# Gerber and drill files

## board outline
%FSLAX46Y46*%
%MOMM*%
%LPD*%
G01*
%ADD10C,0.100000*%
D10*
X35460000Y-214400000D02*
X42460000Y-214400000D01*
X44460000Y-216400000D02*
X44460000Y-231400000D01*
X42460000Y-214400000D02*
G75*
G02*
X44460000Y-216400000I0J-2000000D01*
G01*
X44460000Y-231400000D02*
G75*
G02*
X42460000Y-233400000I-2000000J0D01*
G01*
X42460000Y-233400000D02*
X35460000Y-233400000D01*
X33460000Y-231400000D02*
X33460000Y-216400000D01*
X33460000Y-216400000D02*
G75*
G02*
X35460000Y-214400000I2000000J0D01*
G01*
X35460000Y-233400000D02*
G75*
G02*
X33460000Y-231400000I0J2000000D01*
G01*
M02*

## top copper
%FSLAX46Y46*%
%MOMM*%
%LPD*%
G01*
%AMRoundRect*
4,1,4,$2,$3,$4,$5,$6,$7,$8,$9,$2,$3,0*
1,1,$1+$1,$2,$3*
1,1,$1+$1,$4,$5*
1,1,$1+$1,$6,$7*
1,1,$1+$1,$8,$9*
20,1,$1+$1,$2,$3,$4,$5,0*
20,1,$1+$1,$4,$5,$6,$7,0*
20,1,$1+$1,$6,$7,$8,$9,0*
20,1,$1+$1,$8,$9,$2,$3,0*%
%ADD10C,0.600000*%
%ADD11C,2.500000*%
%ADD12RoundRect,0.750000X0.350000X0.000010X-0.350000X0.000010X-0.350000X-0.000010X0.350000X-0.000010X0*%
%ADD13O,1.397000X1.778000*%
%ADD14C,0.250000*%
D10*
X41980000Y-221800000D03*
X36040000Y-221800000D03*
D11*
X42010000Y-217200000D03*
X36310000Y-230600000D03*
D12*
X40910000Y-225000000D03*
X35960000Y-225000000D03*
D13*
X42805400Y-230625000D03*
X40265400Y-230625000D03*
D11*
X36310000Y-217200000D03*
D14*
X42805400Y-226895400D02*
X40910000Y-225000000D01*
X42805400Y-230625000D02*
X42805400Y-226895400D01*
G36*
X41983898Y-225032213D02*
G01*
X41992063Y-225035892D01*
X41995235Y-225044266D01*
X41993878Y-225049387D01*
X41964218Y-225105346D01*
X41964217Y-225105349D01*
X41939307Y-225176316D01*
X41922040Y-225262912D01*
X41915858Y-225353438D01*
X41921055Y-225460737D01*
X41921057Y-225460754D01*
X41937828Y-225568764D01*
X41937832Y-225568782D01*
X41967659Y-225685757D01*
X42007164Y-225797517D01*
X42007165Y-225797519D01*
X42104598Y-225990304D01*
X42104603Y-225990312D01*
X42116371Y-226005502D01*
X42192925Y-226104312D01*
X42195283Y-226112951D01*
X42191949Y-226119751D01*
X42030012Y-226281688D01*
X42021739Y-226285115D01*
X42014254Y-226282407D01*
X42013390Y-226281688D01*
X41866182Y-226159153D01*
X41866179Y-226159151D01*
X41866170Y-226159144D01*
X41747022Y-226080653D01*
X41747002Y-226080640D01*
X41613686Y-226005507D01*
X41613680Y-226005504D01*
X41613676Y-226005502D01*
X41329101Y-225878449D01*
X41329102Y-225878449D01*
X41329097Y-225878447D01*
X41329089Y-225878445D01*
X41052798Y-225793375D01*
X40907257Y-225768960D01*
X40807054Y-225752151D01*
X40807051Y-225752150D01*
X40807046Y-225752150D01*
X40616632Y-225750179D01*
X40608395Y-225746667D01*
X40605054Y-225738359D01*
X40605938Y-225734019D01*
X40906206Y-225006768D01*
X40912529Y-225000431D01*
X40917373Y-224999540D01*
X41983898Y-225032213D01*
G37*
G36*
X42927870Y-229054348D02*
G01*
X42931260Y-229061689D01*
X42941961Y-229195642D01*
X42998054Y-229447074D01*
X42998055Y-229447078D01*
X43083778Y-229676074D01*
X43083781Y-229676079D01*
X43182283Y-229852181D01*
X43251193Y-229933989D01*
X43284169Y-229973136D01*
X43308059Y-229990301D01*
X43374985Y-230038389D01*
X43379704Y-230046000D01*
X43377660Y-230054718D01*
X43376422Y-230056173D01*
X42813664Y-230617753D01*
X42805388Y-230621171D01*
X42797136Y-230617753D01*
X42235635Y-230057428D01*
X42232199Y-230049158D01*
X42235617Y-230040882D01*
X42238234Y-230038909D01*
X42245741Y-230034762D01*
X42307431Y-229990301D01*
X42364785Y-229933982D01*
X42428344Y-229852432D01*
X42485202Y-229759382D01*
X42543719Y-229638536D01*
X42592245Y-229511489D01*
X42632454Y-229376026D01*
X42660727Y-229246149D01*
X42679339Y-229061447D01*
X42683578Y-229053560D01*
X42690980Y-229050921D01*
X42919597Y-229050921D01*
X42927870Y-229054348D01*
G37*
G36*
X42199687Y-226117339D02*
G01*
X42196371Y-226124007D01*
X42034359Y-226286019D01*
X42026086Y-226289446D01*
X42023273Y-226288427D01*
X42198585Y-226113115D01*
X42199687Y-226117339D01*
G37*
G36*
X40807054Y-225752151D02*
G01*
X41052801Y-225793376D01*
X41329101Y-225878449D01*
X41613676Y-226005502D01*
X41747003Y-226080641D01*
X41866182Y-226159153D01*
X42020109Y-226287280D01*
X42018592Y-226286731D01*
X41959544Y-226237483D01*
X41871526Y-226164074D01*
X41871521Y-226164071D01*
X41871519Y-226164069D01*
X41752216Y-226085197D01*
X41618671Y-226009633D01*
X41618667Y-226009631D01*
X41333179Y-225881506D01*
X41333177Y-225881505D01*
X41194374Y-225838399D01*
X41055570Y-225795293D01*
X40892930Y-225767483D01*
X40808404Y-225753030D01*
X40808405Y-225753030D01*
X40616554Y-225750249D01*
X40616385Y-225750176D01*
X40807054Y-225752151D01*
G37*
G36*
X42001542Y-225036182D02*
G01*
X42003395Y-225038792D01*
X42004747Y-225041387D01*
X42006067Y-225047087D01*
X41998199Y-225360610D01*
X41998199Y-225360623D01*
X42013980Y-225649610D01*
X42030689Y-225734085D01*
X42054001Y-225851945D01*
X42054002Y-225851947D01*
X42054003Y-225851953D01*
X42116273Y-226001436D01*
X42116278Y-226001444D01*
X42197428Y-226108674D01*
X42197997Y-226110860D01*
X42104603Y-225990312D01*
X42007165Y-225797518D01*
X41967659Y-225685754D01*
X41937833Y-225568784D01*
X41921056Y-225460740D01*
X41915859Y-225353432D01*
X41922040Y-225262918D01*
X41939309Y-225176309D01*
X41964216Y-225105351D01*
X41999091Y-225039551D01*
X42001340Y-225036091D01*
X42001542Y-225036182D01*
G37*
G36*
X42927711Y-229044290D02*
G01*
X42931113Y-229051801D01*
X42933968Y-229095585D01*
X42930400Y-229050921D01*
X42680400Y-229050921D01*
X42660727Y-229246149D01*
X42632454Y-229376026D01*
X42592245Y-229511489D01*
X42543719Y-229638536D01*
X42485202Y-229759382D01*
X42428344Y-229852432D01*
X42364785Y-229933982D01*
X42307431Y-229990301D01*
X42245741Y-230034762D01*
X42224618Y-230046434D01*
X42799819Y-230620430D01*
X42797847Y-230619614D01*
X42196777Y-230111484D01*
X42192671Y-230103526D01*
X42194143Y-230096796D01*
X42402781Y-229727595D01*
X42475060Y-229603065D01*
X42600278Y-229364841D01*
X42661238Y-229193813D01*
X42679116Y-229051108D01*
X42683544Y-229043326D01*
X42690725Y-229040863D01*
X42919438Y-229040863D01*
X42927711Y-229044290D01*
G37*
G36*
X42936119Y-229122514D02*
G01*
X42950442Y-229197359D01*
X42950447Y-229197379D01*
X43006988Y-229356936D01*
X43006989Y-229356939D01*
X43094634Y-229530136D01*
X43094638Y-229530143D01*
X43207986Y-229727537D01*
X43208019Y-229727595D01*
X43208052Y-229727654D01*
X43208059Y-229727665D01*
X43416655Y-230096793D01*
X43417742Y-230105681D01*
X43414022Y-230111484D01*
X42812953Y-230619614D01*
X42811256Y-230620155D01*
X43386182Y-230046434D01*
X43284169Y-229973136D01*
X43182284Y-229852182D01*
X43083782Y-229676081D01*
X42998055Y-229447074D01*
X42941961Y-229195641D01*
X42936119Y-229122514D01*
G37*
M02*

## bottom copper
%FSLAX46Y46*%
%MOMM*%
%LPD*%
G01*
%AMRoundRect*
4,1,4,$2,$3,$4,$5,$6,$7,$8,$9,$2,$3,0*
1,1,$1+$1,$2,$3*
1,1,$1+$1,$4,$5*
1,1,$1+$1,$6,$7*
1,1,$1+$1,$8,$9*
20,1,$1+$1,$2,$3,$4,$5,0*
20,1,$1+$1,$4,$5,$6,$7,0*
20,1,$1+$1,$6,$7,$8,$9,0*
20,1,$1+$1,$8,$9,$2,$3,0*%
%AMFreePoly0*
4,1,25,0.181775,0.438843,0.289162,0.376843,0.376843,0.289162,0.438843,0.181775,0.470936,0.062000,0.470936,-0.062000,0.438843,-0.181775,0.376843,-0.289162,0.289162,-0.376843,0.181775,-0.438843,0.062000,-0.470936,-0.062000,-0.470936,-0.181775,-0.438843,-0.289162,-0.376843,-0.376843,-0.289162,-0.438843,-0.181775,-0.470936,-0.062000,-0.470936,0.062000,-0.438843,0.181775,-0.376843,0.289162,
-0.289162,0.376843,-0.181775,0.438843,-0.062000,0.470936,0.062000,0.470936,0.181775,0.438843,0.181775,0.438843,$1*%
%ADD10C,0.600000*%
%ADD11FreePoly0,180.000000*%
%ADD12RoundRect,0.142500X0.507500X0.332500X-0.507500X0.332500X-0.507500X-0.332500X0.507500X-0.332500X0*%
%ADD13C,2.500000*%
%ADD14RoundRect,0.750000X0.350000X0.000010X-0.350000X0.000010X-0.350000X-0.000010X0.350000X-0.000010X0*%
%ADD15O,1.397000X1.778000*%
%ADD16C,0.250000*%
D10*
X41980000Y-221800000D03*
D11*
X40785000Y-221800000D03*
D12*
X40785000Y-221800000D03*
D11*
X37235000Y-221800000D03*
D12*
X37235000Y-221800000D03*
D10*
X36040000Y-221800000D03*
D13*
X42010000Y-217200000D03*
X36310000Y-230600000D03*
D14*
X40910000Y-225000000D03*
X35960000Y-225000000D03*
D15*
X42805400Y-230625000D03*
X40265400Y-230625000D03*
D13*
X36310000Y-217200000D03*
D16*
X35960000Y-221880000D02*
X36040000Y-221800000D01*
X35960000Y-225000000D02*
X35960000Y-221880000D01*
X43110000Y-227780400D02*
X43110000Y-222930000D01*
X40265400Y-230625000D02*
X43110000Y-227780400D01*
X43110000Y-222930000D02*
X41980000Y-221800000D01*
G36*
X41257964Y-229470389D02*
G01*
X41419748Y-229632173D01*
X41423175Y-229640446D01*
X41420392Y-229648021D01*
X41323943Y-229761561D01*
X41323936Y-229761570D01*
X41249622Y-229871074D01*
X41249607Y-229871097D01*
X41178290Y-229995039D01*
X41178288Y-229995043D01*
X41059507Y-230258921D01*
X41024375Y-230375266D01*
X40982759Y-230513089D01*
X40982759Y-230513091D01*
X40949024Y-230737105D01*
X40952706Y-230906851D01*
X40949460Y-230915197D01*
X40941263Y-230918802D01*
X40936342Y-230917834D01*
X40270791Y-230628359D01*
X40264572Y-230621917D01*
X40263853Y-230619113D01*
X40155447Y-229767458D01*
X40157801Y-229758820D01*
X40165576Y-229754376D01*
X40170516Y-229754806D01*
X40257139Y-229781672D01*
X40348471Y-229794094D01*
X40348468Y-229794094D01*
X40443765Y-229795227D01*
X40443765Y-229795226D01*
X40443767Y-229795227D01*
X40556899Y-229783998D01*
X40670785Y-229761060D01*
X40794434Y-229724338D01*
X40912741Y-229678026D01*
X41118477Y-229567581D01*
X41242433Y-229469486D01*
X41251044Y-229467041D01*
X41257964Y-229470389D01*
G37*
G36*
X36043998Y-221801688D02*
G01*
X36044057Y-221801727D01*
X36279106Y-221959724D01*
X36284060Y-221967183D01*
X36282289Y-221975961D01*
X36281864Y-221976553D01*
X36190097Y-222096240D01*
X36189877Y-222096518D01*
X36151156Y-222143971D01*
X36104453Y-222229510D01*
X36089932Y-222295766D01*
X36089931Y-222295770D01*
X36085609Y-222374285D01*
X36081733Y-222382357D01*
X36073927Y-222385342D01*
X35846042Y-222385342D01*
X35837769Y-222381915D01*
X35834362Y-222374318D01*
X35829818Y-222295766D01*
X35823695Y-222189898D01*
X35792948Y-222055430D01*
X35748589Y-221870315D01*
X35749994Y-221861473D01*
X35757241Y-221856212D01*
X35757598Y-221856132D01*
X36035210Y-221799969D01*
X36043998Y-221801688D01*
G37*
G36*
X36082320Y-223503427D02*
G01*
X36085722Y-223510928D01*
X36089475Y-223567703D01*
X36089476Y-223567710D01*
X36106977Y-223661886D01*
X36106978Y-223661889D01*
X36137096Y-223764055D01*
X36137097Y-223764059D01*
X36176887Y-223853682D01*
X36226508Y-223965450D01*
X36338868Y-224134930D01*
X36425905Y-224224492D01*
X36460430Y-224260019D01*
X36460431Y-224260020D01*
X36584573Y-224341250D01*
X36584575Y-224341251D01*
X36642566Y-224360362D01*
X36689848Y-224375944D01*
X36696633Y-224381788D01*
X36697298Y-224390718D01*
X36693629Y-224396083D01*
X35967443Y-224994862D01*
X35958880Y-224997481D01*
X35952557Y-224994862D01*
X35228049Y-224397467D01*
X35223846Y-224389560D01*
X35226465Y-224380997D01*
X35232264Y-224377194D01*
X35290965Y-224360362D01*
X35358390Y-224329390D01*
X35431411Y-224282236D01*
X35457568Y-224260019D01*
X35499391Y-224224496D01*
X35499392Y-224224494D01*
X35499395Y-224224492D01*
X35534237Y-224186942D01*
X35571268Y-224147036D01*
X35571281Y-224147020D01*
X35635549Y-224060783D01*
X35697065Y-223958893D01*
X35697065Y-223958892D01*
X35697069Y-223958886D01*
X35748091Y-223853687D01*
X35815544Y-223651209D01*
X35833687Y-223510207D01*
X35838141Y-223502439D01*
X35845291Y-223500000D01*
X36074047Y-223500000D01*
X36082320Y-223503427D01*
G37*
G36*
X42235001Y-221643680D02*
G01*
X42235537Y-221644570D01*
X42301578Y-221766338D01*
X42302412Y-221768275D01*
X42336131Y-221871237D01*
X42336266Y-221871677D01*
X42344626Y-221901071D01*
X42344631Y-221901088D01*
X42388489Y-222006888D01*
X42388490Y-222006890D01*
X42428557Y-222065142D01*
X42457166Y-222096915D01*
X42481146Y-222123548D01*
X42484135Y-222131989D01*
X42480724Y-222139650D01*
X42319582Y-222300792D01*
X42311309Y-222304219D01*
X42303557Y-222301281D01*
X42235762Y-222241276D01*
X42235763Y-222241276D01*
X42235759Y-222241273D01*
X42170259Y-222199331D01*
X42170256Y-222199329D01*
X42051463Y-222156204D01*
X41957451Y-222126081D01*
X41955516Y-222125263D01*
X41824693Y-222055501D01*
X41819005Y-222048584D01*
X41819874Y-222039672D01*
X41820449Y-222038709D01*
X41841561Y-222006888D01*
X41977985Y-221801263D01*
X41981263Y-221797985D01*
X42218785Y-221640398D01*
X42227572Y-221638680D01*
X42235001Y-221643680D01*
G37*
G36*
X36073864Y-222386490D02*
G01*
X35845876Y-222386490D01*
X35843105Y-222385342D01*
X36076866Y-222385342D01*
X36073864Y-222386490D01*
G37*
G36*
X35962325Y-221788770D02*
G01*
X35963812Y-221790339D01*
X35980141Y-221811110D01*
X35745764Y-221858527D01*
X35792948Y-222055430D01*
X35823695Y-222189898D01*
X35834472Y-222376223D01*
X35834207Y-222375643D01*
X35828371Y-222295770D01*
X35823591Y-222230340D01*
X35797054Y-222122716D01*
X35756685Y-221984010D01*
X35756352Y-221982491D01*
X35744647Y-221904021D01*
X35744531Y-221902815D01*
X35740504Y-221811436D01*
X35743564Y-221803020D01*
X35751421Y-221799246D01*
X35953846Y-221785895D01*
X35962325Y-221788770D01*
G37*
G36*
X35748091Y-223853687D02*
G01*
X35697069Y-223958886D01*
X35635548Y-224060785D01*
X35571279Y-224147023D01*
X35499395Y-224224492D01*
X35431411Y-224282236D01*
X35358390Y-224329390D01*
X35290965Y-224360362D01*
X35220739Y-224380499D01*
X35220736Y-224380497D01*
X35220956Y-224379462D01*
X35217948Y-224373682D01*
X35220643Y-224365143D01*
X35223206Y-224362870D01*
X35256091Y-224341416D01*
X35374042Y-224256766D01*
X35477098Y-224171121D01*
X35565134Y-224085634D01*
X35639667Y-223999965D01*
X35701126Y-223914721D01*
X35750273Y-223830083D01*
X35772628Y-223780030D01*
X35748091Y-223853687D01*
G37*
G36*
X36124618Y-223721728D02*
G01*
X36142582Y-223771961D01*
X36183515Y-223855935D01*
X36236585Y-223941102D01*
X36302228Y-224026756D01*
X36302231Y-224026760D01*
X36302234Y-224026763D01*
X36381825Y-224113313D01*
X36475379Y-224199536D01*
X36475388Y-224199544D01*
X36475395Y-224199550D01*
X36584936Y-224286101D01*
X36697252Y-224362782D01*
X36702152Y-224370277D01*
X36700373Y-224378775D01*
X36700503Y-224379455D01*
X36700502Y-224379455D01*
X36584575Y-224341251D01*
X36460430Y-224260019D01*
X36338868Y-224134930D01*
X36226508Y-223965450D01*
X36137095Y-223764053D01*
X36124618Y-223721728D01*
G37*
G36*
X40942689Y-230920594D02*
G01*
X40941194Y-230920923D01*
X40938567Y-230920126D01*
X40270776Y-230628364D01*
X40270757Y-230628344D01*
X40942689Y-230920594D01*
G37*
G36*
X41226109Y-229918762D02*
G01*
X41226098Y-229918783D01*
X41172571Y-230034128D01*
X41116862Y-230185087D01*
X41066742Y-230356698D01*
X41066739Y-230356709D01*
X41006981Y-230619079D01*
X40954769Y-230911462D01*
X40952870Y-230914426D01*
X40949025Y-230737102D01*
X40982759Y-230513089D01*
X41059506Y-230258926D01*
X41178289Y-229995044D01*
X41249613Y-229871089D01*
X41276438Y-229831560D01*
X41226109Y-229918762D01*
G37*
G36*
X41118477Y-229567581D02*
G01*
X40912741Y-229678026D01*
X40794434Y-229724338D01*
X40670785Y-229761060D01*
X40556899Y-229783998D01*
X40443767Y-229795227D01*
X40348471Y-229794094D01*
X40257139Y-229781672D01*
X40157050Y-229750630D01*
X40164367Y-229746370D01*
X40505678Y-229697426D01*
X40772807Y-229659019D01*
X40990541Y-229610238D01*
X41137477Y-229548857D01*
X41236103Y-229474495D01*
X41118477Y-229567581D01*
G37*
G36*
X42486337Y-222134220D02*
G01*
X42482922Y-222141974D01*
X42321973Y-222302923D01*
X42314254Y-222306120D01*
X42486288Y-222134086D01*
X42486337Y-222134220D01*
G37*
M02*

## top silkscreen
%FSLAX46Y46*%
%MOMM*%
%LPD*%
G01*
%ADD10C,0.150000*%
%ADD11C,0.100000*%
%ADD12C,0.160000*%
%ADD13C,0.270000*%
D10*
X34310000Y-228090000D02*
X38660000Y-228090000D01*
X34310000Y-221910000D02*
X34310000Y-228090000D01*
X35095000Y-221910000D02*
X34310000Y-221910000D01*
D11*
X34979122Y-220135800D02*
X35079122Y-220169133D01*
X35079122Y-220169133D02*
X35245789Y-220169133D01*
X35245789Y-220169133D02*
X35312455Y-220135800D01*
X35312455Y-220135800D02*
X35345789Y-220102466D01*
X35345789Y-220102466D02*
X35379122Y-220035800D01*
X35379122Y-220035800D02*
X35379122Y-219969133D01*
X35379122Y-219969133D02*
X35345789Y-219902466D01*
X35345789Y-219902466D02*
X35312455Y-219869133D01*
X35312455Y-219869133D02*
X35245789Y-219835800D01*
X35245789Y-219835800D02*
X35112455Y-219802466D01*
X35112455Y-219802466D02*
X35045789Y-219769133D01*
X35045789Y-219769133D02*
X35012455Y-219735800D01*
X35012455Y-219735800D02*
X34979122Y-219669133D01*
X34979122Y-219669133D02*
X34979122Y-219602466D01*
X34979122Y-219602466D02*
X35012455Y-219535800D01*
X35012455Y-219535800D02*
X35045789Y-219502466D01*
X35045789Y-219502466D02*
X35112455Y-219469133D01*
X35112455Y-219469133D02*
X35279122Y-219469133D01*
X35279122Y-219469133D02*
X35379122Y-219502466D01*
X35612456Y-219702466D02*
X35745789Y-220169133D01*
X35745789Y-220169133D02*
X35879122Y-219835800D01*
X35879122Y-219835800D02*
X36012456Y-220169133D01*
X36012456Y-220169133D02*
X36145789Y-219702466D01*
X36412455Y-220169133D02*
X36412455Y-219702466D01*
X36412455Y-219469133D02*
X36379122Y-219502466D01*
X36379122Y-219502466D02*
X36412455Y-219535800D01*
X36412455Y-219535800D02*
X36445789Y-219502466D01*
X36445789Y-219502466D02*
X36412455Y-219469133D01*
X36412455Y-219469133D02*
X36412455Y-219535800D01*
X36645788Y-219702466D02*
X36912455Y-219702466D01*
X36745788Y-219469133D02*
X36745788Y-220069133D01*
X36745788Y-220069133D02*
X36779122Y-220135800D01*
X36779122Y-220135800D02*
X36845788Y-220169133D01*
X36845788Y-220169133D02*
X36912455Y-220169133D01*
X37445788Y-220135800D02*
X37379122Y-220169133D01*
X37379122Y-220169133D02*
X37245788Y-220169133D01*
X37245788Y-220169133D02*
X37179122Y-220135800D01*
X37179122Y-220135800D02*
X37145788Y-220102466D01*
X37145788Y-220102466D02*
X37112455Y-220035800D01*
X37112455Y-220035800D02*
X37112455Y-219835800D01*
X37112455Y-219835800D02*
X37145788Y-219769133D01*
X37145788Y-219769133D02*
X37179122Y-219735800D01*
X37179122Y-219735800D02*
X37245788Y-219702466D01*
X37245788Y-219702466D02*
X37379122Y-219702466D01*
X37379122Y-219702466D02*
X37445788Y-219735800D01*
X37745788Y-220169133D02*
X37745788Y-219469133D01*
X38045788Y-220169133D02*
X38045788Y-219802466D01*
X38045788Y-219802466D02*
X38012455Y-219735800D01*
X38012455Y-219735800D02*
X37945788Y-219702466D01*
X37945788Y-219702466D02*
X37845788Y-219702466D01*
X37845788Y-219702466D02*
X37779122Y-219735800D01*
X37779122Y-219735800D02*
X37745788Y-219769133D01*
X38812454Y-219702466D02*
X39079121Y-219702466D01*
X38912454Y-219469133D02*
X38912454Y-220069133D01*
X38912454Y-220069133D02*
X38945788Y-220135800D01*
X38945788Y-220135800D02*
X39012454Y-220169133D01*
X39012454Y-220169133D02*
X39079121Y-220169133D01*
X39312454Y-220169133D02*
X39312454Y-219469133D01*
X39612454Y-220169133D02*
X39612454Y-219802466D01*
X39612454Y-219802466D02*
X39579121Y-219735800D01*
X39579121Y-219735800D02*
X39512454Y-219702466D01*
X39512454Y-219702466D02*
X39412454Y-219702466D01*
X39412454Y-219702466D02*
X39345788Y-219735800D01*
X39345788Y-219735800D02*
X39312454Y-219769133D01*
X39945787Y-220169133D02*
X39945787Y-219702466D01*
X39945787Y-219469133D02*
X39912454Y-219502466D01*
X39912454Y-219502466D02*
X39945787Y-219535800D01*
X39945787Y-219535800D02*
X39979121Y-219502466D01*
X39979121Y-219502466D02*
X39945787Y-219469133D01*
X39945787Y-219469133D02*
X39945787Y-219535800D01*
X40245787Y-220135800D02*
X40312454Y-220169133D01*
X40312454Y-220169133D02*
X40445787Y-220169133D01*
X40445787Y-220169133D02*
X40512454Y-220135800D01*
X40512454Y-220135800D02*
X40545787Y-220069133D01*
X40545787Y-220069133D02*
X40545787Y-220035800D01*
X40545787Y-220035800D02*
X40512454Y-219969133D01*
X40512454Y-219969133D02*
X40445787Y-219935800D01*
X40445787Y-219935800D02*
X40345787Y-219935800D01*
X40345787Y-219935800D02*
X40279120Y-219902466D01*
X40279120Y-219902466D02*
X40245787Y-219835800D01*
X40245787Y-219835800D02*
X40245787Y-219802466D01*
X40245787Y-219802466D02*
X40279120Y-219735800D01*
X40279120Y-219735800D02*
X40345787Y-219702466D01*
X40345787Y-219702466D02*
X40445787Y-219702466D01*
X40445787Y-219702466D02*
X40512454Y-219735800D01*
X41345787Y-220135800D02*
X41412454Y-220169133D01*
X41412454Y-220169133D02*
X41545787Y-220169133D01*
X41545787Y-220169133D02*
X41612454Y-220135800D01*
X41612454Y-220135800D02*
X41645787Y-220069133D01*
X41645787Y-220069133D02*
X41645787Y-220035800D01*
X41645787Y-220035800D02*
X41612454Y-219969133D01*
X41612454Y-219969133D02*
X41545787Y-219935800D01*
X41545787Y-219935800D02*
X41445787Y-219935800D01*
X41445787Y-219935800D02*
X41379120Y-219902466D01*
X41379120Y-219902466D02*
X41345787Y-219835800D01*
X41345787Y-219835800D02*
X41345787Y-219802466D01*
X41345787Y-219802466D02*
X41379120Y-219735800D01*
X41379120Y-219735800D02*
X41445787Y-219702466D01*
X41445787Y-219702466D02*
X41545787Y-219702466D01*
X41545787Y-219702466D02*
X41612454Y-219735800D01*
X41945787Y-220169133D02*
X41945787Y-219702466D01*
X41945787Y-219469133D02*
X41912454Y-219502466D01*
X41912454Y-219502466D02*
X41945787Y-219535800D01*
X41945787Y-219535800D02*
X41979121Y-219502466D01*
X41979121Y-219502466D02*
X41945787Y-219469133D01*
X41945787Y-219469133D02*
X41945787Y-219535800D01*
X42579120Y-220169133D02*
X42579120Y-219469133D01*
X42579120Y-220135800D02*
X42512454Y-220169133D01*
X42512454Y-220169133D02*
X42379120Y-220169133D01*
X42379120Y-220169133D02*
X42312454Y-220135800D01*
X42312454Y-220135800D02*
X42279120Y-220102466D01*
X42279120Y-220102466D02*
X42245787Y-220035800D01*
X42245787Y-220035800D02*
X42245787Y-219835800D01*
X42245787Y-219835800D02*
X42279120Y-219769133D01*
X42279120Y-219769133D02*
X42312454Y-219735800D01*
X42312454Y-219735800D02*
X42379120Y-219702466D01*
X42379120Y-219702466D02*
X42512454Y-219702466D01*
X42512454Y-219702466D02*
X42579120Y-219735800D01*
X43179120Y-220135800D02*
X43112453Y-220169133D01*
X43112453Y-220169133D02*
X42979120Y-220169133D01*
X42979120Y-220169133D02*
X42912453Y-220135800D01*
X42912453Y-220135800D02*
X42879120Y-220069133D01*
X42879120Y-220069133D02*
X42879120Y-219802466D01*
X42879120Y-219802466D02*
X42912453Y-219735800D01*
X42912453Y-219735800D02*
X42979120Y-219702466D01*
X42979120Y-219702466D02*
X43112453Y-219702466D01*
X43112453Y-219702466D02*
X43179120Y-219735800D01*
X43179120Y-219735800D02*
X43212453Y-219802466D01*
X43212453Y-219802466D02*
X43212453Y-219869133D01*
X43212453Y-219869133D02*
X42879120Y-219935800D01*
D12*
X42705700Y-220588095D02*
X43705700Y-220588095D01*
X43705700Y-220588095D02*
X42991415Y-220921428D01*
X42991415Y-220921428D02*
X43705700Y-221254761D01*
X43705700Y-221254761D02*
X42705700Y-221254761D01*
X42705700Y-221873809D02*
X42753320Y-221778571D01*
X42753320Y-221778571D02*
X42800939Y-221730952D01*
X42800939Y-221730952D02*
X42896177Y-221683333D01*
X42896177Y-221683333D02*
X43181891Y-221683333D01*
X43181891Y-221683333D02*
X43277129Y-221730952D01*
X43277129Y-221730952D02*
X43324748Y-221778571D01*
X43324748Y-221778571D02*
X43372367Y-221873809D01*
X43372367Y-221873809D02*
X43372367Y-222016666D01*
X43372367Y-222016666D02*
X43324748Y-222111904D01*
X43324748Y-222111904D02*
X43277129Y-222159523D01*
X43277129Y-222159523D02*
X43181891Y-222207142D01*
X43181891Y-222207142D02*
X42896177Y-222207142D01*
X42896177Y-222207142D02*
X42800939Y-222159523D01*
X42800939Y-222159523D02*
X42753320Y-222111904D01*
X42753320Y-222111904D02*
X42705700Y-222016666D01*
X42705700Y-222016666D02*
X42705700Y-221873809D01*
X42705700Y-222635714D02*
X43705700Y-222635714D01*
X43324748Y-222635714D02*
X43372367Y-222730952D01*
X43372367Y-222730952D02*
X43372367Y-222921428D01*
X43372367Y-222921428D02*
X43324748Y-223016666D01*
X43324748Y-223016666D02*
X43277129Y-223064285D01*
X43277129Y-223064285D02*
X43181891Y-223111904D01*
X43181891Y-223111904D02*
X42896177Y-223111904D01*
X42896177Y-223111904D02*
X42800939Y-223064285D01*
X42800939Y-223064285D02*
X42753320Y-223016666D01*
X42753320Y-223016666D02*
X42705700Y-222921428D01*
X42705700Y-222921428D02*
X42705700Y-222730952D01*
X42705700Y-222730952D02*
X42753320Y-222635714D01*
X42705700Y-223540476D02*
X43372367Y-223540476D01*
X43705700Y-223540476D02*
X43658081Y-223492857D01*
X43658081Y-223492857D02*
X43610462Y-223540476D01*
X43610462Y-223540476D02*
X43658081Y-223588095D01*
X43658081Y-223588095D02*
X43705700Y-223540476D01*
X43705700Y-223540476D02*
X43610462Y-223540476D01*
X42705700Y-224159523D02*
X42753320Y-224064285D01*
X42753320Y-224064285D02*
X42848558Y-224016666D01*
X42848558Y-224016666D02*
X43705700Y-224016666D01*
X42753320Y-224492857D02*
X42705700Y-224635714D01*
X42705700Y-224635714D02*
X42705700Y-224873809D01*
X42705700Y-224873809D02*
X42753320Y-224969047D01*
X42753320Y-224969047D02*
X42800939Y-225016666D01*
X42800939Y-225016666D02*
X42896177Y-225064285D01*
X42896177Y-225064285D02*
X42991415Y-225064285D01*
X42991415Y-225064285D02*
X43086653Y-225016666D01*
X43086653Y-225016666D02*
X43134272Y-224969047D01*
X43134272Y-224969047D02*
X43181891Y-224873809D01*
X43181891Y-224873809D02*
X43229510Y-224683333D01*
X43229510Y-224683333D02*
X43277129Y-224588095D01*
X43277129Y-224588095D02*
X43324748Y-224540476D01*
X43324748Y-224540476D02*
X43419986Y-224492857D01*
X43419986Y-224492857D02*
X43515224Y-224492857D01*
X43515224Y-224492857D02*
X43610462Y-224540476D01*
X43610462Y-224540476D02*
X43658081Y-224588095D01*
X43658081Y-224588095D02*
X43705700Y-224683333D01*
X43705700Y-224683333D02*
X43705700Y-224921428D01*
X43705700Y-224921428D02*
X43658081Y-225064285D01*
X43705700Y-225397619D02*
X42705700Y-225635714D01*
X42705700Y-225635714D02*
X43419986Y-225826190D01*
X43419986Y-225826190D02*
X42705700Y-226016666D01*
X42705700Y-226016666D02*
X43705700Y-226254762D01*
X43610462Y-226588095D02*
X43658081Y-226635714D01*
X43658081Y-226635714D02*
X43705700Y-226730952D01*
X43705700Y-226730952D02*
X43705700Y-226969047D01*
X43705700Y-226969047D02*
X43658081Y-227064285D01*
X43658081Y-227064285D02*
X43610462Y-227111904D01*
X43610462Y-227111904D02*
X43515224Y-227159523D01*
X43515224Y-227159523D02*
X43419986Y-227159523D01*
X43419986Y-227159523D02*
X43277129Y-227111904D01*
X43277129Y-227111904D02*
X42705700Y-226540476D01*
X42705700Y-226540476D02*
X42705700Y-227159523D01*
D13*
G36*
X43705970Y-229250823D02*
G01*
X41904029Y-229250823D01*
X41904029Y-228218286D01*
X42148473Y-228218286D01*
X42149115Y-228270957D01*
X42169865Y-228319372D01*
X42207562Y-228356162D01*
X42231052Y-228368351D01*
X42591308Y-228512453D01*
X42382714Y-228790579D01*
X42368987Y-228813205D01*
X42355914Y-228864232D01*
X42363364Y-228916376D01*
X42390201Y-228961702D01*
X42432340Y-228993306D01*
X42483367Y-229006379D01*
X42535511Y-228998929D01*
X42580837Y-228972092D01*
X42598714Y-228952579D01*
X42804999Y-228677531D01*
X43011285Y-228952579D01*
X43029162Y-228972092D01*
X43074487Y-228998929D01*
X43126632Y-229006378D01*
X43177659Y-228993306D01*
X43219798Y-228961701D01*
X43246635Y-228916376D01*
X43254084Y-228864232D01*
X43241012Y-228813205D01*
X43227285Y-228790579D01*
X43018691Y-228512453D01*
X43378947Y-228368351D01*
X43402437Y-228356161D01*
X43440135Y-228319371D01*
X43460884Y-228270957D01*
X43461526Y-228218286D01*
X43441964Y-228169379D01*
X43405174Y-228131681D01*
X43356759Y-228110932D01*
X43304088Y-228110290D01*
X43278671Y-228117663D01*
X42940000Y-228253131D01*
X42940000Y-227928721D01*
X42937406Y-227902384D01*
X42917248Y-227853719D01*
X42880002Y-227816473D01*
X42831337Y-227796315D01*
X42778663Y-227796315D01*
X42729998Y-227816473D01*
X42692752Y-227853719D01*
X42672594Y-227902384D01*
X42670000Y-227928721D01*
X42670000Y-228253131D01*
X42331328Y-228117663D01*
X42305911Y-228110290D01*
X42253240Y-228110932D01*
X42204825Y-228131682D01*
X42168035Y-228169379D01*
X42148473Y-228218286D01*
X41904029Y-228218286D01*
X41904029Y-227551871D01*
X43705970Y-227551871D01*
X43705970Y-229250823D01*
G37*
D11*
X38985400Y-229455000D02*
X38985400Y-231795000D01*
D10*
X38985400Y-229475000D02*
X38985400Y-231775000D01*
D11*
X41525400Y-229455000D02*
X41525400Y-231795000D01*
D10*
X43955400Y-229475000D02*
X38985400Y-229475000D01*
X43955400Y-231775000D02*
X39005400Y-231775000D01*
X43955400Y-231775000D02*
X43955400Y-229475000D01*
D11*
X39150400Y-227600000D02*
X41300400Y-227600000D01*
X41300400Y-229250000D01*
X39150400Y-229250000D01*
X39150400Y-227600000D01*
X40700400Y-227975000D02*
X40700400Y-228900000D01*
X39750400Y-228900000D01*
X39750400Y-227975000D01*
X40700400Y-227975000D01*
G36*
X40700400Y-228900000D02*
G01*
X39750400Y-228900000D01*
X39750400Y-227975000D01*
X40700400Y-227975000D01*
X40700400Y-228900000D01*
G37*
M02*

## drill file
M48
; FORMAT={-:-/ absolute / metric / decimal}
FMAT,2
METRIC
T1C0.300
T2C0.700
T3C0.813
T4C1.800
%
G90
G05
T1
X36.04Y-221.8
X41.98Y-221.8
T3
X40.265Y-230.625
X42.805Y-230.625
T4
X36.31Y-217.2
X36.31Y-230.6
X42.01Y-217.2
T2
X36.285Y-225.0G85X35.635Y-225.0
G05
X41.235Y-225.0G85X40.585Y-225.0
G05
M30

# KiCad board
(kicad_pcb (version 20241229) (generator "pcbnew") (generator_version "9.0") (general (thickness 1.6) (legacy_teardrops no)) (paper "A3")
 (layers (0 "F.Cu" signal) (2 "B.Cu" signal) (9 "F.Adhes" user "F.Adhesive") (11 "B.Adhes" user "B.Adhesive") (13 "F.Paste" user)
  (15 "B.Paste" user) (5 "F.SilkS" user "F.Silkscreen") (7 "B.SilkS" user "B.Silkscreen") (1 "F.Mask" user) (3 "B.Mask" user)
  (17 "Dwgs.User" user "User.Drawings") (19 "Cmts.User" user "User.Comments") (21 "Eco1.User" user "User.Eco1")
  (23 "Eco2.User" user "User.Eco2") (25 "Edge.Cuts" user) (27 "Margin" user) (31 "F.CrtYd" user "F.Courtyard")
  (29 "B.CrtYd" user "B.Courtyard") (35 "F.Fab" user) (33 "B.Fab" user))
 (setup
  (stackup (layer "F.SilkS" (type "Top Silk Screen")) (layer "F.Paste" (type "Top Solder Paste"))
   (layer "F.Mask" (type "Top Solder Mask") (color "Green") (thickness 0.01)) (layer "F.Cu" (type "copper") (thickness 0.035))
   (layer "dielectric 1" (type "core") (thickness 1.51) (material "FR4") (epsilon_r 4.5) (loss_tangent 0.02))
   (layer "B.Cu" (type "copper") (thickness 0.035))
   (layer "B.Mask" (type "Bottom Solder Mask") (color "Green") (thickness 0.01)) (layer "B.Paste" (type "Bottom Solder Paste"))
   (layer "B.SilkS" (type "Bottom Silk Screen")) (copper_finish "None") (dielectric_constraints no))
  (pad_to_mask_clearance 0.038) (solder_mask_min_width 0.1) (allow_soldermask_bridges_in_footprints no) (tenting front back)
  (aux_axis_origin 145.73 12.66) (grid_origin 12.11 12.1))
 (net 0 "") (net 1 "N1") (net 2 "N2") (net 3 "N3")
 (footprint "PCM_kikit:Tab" (layer "F.Cu") (at 44.71 220.5 180)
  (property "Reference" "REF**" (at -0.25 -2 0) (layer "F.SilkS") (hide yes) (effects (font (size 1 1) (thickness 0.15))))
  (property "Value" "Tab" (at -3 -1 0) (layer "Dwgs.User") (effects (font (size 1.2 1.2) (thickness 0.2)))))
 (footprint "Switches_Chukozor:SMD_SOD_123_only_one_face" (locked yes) (layer "F.Cu") (at 39.01 221.8 180)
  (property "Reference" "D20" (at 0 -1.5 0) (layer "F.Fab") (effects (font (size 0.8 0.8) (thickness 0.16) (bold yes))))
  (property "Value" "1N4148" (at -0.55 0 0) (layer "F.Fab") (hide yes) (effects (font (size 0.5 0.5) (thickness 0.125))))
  (pad "1" thru_hole circle (at -2.97 0 180) (size 0.6 0.6) (drill 0.3) (layers "*.Cu") (remove_unused_layers no) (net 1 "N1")
   (teardrops (best_length_ratio 0.5) (max_length 1) (best_width_ratio 1) (max_width 2) (curved_edges yes) (filter_ratio 0.9) (enabled yes)
    (allow_two_segments yes) (prefer_zone_connections yes)))
  (pad "1" smd custom (at -1.775 0 180) (size 0.95 0.95) (layers "B.Cu") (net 1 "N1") (thermal_bridge_angle 90)
   (options (clearance outline) (anchor circle)) (primitives)
   (teardrops (best_length_ratio 0.5) (max_length 1) (best_width_ratio 1) (max_width 2) (curved_edges no) (filter_ratio 0.9) (enabled no)
    (allow_two_segments no) (prefer_zone_connections yes)))
  (pad "1" smd roundrect (at -1.775 0 180) (size 1.3 0.95) (layers "B.Cu" "B.Mask") (roundrect_rratio 0.15) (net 1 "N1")
   (teardrops (best_length_ratio 0.5) (max_length 1) (best_width_ratio 1) (max_width 2) (curved_edges yes) (filter_ratio 0.9) (enabled yes)
    (allow_two_segments yes) (prefer_zone_connections yes)))
  (pad "2" smd custom (at 1.775 0 180) (size 0.95 0.95) (layers "B.Cu") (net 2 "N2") (thermal_bridge_angle 90)
   (options (clearance outline) (anchor circle)) (primitives)
   (teardrops (best_length_ratio 0.5) (max_length 1) (best_width_ratio 1) (max_width 2) (curved_edges no) (filter_ratio 0.9) (enabled no)
    (allow_two_segments no) (prefer_zone_connections yes)))
  (pad "2" smd roundrect (at 1.775 0 180) (size 1.3 0.95) (layers "B.Cu" "B.Mask") (roundrect_rratio 0.15) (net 2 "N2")
   (teardrops (best_length_ratio 0.5) (max_length 1) (best_width_ratio 1) (max_width 2) (curved_edges yes) (filter_ratio 0.9) (enabled yes)
    (allow_two_segments yes) (prefer_zone_connections yes)))
  (pad "2" thru_hole circle (at 2.97 0 180) (size 0.6 0.6) (drill 0.3) (layers "*.Cu") (remove_unused_layers no) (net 2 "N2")
   (teardrops (best_length_ratio 0.5) (max_length 1) (best_width_ratio 1) (max_width 2) (curved_edges yes) (filter_ratio 0.9) (enabled yes)
    (allow_two_segments yes) (prefer_zone_connections yes))))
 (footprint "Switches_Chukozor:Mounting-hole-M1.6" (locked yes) (layer "F.Cu") (at 42.01 217.2)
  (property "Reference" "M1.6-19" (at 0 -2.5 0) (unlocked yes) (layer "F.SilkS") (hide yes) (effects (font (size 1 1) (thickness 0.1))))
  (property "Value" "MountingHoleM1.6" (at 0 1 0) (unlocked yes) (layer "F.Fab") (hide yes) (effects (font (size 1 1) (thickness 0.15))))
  (pad "" np_thru_hole circle (at 0 0) (size 2.5 2.5) (drill 1.8) (layers "*.Cu" "*.Mask") (clearance 0.2)))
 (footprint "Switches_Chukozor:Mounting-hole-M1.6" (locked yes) (layer "F.Cu") (at 36.31 230.6)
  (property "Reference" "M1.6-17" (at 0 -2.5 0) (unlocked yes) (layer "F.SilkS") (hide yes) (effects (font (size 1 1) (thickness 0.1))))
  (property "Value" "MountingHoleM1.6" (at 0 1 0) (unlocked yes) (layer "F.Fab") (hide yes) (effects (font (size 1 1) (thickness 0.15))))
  (pad "" np_thru_hole circle (at 0 0) (size 2.5 2.5) (drill 1.8) (layers "*.Cu" "*.Mask") (clearance 0.2)))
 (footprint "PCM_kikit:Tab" (layer "F.Cu") (at 39.11 214.15 -90)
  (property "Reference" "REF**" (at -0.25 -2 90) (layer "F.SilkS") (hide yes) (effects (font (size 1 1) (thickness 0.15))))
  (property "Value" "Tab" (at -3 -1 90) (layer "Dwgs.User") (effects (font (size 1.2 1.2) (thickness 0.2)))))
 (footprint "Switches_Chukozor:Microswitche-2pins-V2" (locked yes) (layer "F.Cu") (at 40.91 225 180)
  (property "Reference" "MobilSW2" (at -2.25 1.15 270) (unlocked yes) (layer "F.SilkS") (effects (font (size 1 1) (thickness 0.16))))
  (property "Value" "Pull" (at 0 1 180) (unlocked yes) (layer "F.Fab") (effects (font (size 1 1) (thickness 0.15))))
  (pad "1" thru_hole roundrect (at 0 0 180) (size 2.2 1.5) (drill oval 1.35 0.7) (layers "*.Cu" "*.Mask") (remove_unused_layers no)
   (roundrect_rratio 0.5) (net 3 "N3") (thermal_bridge_angle 45)
   (teardrops (best_length_ratio 0.5) (max_length 1) (best_width_ratio 1) (max_width 2) (curved_edges yes) (filter_ratio 0.9) (enabled yes)
    (allow_two_segments yes) (prefer_zone_connections yes)))
  (pad "2" thru_hole roundrect (at 4.95 0 180) (size 2.2 1.5) (drill oval 1.35 0.7) (layers "*.Cu" "*.Mask") (remove_unused_layers no)
   (roundrect_rratio 0.5) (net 2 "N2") (thermal_bridge_angle 45)
   (teardrops (best_length_ratio 0.5) (max_length 1) (best_width_ratio 1) (max_width 2) (curved_edges yes) (filter_ratio 0.9) (enabled yes)
    (allow_two_segments yes) (prefer_zone_connections yes))))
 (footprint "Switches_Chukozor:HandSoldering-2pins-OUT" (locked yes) (layer "F.Cu") (at 41.41 230.625)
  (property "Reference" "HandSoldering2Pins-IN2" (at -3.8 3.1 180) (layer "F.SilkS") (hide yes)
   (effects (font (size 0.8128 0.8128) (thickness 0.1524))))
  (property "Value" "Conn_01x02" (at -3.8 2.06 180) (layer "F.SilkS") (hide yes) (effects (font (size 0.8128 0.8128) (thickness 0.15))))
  (fp_line (start -2.4246 -1.17) (end -2.4246 1.17) (stroke (width 0.1) (type default)) (layer "F.SilkS"))
  (fp_line (start -2.4246 -1.15) (end -2.4246 1.15) (stroke (width 0.15) (type solid)) (layer "F.SilkS"))
  (fp_line (start 0.1154 -1.17) (end 0.1154 1.17) (stroke (width 0.1) (type default)) (layer "F.SilkS"))
  (fp_line (start 2.5454 -1.15) (end -2.4246 -1.15) (stroke (width 0.15) (type solid)) (layer "F.SilkS"))
  (fp_line (start 2.5454 1.15) (end -2.4046 1.15) (stroke (width 0.15) (type solid)) (layer "F.SilkS"))
  (fp_line (start 2.5454 1.15) (end 2.5454 -1.15) (stroke (width 0.15) (type solid)) (layer "F.SilkS"))
  (fp_rect (start -0.1096 -3.025) (end -2.2596 -1.375) (stroke (width 0.1) (type default)) (fill no) (layer "F.SilkS"))
  (fp_poly
   (pts (xy -0.7096 -2.65) (xy -0.7096 -1.725) (xy -1.6596 -1.725) (xy -1.6596 -2.65)) (stroke (width 0.1) (type solid)) (fill yes)
   (layer "F.SilkS"))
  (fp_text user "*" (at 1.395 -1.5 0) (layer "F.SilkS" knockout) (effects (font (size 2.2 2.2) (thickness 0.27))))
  (pad "1" thru_hole oval (at 1.3954 0) (size 1.397 1.778) (drill 0.8128) (layers "*.Cu" "*.Mask") (remove_unused_layers no) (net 3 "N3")
   (teardrops (best_length_ratio 0.5) (max_length 1) (best_width_ratio 1) (max_width 2) (curved_edges yes) (filter_ratio 0.9) (enabled yes)
    (allow_two_segments yes) (prefer_zone_connections yes)))
  (pad "2" thru_hole oval (at -1.1446 0) (size 1.397 1.778) (drill 0.8128) (layers "*.Cu" "*.Mask") (remove_unused_layers no) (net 1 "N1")
   (teardrops (best_length_ratio 0.5) (max_length 1) (best_width_ratio 1) (max_width 2) (curved_edges yes) (filter_ratio 0.9) (enabled yes)
    (allow_two_segments yes) (prefer_zone_connections yes))))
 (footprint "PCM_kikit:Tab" (layer "F.Cu") (at 39.11 233.65 90)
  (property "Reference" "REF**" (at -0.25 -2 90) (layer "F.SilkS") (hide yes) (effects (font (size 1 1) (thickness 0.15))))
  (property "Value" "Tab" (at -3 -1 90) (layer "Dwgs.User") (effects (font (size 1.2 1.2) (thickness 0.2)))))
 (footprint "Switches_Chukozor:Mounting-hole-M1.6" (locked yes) (layer "F.Cu") (at 36.31 217.2)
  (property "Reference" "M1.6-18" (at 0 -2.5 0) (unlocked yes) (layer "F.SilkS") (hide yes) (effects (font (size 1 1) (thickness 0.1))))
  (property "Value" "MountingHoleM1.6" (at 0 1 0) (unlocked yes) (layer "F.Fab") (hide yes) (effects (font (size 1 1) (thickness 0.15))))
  (pad "" np_thru_hole circle (at 0 0) (size 2.5 2.5) (drill 1.8) (layers "*.Cu" "*.Mask") (clearance 0.2)))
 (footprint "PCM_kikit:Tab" (layer "F.Cu") (at 33.11 220.5)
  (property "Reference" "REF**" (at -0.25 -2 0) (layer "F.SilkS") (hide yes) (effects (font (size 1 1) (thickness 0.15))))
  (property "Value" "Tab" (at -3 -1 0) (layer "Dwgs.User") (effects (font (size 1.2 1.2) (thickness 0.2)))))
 (gr_line (start 34.31 228.09) (end 38.66 228.09) (stroke (width 0.15) (type default)) (layer "F.SilkS"))
 (gr_line (start 34.31 221.91) (end 34.31 228.09) (stroke (width 0.15) (type default)) (layer "F.SilkS"))
 (gr_line (start 35.095 221.91) (end 34.31 221.91) (stroke (width 0.15) (type default)) (layer "F.SilkS"))
 (gr_line (start 35.46 214.4) (end 42.46 214.4) (stroke (width 0.1) (type default)) (locked yes) (layer "Edge.Cuts"))
 (gr_line (start 44.46 216.4) (end 44.46 231.4) (stroke (width 0.1) (type default)) (locked yes) (layer "Edge.Cuts"))
 (gr_arc (start 42.46 214.4) (mid 43.874214 214.985786) (end 44.46 216.4) (stroke (width 0.1) (type default)) (locked yes)
  (layer "Edge.Cuts"))
 (gr_arc (start 44.46 231.4) (mid 43.874214 232.814214) (end 42.46 233.4) (stroke (width 0.1) (type default)) (locked yes)
  (layer "Edge.Cuts"))
 (gr_line (start 42.46 233.4) (end 35.46 233.4) (stroke (width 0.1) (type default)) (locked yes) (layer "Edge.Cuts"))
 (gr_line (start 33.46 231.4) (end 33.46 216.4) (stroke (width 0.1) (type default)) (locked yes) (layer "Edge.Cuts"))
 (gr_arc (start 33.46 216.4) (mid 34.045786 214.985786) (end 35.46 214.4) (stroke (width 0.1) (type default)) (locked yes)
  (layer "Edge.Cuts"))
 (gr_arc (start 35.46 233.4) (mid 34.045786 232.814214) (end 33.46 231.4) (stroke (width 0.1) (type default)) (locked yes)
  (layer "Edge.Cuts"))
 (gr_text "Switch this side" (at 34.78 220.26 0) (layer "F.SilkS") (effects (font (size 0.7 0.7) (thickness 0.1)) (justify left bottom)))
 (segment (start 35.96 221.88) (end 36.04 221.8) (width 0.25) (layer "B.Cu") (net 2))
 (segment (start 35.96 225) (end 35.96 221.88) (width 0.25) (layer "B.Cu") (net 2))
 (segment (start 43.11 227.7804) (end 43.11 222.93) (width 0.25) (layer "B.Cu") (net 1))
 (segment (start 40.2654 230.625) (end 43.11 227.7804) (width 0.25) (layer "B.Cu") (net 1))
 (segment (start 43.11 222.93) (end 41.98 221.8) (width 0.25) (layer "B.Cu") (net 1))
 (segment (start 42.8054 226.8954) (end 40.91 225) (width 0.25) (layer "F.Cu") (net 3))
 (segment (start 42.8054 230.625) (end 42.8054 226.8954) (width 0.25) (layer "F.Cu") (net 3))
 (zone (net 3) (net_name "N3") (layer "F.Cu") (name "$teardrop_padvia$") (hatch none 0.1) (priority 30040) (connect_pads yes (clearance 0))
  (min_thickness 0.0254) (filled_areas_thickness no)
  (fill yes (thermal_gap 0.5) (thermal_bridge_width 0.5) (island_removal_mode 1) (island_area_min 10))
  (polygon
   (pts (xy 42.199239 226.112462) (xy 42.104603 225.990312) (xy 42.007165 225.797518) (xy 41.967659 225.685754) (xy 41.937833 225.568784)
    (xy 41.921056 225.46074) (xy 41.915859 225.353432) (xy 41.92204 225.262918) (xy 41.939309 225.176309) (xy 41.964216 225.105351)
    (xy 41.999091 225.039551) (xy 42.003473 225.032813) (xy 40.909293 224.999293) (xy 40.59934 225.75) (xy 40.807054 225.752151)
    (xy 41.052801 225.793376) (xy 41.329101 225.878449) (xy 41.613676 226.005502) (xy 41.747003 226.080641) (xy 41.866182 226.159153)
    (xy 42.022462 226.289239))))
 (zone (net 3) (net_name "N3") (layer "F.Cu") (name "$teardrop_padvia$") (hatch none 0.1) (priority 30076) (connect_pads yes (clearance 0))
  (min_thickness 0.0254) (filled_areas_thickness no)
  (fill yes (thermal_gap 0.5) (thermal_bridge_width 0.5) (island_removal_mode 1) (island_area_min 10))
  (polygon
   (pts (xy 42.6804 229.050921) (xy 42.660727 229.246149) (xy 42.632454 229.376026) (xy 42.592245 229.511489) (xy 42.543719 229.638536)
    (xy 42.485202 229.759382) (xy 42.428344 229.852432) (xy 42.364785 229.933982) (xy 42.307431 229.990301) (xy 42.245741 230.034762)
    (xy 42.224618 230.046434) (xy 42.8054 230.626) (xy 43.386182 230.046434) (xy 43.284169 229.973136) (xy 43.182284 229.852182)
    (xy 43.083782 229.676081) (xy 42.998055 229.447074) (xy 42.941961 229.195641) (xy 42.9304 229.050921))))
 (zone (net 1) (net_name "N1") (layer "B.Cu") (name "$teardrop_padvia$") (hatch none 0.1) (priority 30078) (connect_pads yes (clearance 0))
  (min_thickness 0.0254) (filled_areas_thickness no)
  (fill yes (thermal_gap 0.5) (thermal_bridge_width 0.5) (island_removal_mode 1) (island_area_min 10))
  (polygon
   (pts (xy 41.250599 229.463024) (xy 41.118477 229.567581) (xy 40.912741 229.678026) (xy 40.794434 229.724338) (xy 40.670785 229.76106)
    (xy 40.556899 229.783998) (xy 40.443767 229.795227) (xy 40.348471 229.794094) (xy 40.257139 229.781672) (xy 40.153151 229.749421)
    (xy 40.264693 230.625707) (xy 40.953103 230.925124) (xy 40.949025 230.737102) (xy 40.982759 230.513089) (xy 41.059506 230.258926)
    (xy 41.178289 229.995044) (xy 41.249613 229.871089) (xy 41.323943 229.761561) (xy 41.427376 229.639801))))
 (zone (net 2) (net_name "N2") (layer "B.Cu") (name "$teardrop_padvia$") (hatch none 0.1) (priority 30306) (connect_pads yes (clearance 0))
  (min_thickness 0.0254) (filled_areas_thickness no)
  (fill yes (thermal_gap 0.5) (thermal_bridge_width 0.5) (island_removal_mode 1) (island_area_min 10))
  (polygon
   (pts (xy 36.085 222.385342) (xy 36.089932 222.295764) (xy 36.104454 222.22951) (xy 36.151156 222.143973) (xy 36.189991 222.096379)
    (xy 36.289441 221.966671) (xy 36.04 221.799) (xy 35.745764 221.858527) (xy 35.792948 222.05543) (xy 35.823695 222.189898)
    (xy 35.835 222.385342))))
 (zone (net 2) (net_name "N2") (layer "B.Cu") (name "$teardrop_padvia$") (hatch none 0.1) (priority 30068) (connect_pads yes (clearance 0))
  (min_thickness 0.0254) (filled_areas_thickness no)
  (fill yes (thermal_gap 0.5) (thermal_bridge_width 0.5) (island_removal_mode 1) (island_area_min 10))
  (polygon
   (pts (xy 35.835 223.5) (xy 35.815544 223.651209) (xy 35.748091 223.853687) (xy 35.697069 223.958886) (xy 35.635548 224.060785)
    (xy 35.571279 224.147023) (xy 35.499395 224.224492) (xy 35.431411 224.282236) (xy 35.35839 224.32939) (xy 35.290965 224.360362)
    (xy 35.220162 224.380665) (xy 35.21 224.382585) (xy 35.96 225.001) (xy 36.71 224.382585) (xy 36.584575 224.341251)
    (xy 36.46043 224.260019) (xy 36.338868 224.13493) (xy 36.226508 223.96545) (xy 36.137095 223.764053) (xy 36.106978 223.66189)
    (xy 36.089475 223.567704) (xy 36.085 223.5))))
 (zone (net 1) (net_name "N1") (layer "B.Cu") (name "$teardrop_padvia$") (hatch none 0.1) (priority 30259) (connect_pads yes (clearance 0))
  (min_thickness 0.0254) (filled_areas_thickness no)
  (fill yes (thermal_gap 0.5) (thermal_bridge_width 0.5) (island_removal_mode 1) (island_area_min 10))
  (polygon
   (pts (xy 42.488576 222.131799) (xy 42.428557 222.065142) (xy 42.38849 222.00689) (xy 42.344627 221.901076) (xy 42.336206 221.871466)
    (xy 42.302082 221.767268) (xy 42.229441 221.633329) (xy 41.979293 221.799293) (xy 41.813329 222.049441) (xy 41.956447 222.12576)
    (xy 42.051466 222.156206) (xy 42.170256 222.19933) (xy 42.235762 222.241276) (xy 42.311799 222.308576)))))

